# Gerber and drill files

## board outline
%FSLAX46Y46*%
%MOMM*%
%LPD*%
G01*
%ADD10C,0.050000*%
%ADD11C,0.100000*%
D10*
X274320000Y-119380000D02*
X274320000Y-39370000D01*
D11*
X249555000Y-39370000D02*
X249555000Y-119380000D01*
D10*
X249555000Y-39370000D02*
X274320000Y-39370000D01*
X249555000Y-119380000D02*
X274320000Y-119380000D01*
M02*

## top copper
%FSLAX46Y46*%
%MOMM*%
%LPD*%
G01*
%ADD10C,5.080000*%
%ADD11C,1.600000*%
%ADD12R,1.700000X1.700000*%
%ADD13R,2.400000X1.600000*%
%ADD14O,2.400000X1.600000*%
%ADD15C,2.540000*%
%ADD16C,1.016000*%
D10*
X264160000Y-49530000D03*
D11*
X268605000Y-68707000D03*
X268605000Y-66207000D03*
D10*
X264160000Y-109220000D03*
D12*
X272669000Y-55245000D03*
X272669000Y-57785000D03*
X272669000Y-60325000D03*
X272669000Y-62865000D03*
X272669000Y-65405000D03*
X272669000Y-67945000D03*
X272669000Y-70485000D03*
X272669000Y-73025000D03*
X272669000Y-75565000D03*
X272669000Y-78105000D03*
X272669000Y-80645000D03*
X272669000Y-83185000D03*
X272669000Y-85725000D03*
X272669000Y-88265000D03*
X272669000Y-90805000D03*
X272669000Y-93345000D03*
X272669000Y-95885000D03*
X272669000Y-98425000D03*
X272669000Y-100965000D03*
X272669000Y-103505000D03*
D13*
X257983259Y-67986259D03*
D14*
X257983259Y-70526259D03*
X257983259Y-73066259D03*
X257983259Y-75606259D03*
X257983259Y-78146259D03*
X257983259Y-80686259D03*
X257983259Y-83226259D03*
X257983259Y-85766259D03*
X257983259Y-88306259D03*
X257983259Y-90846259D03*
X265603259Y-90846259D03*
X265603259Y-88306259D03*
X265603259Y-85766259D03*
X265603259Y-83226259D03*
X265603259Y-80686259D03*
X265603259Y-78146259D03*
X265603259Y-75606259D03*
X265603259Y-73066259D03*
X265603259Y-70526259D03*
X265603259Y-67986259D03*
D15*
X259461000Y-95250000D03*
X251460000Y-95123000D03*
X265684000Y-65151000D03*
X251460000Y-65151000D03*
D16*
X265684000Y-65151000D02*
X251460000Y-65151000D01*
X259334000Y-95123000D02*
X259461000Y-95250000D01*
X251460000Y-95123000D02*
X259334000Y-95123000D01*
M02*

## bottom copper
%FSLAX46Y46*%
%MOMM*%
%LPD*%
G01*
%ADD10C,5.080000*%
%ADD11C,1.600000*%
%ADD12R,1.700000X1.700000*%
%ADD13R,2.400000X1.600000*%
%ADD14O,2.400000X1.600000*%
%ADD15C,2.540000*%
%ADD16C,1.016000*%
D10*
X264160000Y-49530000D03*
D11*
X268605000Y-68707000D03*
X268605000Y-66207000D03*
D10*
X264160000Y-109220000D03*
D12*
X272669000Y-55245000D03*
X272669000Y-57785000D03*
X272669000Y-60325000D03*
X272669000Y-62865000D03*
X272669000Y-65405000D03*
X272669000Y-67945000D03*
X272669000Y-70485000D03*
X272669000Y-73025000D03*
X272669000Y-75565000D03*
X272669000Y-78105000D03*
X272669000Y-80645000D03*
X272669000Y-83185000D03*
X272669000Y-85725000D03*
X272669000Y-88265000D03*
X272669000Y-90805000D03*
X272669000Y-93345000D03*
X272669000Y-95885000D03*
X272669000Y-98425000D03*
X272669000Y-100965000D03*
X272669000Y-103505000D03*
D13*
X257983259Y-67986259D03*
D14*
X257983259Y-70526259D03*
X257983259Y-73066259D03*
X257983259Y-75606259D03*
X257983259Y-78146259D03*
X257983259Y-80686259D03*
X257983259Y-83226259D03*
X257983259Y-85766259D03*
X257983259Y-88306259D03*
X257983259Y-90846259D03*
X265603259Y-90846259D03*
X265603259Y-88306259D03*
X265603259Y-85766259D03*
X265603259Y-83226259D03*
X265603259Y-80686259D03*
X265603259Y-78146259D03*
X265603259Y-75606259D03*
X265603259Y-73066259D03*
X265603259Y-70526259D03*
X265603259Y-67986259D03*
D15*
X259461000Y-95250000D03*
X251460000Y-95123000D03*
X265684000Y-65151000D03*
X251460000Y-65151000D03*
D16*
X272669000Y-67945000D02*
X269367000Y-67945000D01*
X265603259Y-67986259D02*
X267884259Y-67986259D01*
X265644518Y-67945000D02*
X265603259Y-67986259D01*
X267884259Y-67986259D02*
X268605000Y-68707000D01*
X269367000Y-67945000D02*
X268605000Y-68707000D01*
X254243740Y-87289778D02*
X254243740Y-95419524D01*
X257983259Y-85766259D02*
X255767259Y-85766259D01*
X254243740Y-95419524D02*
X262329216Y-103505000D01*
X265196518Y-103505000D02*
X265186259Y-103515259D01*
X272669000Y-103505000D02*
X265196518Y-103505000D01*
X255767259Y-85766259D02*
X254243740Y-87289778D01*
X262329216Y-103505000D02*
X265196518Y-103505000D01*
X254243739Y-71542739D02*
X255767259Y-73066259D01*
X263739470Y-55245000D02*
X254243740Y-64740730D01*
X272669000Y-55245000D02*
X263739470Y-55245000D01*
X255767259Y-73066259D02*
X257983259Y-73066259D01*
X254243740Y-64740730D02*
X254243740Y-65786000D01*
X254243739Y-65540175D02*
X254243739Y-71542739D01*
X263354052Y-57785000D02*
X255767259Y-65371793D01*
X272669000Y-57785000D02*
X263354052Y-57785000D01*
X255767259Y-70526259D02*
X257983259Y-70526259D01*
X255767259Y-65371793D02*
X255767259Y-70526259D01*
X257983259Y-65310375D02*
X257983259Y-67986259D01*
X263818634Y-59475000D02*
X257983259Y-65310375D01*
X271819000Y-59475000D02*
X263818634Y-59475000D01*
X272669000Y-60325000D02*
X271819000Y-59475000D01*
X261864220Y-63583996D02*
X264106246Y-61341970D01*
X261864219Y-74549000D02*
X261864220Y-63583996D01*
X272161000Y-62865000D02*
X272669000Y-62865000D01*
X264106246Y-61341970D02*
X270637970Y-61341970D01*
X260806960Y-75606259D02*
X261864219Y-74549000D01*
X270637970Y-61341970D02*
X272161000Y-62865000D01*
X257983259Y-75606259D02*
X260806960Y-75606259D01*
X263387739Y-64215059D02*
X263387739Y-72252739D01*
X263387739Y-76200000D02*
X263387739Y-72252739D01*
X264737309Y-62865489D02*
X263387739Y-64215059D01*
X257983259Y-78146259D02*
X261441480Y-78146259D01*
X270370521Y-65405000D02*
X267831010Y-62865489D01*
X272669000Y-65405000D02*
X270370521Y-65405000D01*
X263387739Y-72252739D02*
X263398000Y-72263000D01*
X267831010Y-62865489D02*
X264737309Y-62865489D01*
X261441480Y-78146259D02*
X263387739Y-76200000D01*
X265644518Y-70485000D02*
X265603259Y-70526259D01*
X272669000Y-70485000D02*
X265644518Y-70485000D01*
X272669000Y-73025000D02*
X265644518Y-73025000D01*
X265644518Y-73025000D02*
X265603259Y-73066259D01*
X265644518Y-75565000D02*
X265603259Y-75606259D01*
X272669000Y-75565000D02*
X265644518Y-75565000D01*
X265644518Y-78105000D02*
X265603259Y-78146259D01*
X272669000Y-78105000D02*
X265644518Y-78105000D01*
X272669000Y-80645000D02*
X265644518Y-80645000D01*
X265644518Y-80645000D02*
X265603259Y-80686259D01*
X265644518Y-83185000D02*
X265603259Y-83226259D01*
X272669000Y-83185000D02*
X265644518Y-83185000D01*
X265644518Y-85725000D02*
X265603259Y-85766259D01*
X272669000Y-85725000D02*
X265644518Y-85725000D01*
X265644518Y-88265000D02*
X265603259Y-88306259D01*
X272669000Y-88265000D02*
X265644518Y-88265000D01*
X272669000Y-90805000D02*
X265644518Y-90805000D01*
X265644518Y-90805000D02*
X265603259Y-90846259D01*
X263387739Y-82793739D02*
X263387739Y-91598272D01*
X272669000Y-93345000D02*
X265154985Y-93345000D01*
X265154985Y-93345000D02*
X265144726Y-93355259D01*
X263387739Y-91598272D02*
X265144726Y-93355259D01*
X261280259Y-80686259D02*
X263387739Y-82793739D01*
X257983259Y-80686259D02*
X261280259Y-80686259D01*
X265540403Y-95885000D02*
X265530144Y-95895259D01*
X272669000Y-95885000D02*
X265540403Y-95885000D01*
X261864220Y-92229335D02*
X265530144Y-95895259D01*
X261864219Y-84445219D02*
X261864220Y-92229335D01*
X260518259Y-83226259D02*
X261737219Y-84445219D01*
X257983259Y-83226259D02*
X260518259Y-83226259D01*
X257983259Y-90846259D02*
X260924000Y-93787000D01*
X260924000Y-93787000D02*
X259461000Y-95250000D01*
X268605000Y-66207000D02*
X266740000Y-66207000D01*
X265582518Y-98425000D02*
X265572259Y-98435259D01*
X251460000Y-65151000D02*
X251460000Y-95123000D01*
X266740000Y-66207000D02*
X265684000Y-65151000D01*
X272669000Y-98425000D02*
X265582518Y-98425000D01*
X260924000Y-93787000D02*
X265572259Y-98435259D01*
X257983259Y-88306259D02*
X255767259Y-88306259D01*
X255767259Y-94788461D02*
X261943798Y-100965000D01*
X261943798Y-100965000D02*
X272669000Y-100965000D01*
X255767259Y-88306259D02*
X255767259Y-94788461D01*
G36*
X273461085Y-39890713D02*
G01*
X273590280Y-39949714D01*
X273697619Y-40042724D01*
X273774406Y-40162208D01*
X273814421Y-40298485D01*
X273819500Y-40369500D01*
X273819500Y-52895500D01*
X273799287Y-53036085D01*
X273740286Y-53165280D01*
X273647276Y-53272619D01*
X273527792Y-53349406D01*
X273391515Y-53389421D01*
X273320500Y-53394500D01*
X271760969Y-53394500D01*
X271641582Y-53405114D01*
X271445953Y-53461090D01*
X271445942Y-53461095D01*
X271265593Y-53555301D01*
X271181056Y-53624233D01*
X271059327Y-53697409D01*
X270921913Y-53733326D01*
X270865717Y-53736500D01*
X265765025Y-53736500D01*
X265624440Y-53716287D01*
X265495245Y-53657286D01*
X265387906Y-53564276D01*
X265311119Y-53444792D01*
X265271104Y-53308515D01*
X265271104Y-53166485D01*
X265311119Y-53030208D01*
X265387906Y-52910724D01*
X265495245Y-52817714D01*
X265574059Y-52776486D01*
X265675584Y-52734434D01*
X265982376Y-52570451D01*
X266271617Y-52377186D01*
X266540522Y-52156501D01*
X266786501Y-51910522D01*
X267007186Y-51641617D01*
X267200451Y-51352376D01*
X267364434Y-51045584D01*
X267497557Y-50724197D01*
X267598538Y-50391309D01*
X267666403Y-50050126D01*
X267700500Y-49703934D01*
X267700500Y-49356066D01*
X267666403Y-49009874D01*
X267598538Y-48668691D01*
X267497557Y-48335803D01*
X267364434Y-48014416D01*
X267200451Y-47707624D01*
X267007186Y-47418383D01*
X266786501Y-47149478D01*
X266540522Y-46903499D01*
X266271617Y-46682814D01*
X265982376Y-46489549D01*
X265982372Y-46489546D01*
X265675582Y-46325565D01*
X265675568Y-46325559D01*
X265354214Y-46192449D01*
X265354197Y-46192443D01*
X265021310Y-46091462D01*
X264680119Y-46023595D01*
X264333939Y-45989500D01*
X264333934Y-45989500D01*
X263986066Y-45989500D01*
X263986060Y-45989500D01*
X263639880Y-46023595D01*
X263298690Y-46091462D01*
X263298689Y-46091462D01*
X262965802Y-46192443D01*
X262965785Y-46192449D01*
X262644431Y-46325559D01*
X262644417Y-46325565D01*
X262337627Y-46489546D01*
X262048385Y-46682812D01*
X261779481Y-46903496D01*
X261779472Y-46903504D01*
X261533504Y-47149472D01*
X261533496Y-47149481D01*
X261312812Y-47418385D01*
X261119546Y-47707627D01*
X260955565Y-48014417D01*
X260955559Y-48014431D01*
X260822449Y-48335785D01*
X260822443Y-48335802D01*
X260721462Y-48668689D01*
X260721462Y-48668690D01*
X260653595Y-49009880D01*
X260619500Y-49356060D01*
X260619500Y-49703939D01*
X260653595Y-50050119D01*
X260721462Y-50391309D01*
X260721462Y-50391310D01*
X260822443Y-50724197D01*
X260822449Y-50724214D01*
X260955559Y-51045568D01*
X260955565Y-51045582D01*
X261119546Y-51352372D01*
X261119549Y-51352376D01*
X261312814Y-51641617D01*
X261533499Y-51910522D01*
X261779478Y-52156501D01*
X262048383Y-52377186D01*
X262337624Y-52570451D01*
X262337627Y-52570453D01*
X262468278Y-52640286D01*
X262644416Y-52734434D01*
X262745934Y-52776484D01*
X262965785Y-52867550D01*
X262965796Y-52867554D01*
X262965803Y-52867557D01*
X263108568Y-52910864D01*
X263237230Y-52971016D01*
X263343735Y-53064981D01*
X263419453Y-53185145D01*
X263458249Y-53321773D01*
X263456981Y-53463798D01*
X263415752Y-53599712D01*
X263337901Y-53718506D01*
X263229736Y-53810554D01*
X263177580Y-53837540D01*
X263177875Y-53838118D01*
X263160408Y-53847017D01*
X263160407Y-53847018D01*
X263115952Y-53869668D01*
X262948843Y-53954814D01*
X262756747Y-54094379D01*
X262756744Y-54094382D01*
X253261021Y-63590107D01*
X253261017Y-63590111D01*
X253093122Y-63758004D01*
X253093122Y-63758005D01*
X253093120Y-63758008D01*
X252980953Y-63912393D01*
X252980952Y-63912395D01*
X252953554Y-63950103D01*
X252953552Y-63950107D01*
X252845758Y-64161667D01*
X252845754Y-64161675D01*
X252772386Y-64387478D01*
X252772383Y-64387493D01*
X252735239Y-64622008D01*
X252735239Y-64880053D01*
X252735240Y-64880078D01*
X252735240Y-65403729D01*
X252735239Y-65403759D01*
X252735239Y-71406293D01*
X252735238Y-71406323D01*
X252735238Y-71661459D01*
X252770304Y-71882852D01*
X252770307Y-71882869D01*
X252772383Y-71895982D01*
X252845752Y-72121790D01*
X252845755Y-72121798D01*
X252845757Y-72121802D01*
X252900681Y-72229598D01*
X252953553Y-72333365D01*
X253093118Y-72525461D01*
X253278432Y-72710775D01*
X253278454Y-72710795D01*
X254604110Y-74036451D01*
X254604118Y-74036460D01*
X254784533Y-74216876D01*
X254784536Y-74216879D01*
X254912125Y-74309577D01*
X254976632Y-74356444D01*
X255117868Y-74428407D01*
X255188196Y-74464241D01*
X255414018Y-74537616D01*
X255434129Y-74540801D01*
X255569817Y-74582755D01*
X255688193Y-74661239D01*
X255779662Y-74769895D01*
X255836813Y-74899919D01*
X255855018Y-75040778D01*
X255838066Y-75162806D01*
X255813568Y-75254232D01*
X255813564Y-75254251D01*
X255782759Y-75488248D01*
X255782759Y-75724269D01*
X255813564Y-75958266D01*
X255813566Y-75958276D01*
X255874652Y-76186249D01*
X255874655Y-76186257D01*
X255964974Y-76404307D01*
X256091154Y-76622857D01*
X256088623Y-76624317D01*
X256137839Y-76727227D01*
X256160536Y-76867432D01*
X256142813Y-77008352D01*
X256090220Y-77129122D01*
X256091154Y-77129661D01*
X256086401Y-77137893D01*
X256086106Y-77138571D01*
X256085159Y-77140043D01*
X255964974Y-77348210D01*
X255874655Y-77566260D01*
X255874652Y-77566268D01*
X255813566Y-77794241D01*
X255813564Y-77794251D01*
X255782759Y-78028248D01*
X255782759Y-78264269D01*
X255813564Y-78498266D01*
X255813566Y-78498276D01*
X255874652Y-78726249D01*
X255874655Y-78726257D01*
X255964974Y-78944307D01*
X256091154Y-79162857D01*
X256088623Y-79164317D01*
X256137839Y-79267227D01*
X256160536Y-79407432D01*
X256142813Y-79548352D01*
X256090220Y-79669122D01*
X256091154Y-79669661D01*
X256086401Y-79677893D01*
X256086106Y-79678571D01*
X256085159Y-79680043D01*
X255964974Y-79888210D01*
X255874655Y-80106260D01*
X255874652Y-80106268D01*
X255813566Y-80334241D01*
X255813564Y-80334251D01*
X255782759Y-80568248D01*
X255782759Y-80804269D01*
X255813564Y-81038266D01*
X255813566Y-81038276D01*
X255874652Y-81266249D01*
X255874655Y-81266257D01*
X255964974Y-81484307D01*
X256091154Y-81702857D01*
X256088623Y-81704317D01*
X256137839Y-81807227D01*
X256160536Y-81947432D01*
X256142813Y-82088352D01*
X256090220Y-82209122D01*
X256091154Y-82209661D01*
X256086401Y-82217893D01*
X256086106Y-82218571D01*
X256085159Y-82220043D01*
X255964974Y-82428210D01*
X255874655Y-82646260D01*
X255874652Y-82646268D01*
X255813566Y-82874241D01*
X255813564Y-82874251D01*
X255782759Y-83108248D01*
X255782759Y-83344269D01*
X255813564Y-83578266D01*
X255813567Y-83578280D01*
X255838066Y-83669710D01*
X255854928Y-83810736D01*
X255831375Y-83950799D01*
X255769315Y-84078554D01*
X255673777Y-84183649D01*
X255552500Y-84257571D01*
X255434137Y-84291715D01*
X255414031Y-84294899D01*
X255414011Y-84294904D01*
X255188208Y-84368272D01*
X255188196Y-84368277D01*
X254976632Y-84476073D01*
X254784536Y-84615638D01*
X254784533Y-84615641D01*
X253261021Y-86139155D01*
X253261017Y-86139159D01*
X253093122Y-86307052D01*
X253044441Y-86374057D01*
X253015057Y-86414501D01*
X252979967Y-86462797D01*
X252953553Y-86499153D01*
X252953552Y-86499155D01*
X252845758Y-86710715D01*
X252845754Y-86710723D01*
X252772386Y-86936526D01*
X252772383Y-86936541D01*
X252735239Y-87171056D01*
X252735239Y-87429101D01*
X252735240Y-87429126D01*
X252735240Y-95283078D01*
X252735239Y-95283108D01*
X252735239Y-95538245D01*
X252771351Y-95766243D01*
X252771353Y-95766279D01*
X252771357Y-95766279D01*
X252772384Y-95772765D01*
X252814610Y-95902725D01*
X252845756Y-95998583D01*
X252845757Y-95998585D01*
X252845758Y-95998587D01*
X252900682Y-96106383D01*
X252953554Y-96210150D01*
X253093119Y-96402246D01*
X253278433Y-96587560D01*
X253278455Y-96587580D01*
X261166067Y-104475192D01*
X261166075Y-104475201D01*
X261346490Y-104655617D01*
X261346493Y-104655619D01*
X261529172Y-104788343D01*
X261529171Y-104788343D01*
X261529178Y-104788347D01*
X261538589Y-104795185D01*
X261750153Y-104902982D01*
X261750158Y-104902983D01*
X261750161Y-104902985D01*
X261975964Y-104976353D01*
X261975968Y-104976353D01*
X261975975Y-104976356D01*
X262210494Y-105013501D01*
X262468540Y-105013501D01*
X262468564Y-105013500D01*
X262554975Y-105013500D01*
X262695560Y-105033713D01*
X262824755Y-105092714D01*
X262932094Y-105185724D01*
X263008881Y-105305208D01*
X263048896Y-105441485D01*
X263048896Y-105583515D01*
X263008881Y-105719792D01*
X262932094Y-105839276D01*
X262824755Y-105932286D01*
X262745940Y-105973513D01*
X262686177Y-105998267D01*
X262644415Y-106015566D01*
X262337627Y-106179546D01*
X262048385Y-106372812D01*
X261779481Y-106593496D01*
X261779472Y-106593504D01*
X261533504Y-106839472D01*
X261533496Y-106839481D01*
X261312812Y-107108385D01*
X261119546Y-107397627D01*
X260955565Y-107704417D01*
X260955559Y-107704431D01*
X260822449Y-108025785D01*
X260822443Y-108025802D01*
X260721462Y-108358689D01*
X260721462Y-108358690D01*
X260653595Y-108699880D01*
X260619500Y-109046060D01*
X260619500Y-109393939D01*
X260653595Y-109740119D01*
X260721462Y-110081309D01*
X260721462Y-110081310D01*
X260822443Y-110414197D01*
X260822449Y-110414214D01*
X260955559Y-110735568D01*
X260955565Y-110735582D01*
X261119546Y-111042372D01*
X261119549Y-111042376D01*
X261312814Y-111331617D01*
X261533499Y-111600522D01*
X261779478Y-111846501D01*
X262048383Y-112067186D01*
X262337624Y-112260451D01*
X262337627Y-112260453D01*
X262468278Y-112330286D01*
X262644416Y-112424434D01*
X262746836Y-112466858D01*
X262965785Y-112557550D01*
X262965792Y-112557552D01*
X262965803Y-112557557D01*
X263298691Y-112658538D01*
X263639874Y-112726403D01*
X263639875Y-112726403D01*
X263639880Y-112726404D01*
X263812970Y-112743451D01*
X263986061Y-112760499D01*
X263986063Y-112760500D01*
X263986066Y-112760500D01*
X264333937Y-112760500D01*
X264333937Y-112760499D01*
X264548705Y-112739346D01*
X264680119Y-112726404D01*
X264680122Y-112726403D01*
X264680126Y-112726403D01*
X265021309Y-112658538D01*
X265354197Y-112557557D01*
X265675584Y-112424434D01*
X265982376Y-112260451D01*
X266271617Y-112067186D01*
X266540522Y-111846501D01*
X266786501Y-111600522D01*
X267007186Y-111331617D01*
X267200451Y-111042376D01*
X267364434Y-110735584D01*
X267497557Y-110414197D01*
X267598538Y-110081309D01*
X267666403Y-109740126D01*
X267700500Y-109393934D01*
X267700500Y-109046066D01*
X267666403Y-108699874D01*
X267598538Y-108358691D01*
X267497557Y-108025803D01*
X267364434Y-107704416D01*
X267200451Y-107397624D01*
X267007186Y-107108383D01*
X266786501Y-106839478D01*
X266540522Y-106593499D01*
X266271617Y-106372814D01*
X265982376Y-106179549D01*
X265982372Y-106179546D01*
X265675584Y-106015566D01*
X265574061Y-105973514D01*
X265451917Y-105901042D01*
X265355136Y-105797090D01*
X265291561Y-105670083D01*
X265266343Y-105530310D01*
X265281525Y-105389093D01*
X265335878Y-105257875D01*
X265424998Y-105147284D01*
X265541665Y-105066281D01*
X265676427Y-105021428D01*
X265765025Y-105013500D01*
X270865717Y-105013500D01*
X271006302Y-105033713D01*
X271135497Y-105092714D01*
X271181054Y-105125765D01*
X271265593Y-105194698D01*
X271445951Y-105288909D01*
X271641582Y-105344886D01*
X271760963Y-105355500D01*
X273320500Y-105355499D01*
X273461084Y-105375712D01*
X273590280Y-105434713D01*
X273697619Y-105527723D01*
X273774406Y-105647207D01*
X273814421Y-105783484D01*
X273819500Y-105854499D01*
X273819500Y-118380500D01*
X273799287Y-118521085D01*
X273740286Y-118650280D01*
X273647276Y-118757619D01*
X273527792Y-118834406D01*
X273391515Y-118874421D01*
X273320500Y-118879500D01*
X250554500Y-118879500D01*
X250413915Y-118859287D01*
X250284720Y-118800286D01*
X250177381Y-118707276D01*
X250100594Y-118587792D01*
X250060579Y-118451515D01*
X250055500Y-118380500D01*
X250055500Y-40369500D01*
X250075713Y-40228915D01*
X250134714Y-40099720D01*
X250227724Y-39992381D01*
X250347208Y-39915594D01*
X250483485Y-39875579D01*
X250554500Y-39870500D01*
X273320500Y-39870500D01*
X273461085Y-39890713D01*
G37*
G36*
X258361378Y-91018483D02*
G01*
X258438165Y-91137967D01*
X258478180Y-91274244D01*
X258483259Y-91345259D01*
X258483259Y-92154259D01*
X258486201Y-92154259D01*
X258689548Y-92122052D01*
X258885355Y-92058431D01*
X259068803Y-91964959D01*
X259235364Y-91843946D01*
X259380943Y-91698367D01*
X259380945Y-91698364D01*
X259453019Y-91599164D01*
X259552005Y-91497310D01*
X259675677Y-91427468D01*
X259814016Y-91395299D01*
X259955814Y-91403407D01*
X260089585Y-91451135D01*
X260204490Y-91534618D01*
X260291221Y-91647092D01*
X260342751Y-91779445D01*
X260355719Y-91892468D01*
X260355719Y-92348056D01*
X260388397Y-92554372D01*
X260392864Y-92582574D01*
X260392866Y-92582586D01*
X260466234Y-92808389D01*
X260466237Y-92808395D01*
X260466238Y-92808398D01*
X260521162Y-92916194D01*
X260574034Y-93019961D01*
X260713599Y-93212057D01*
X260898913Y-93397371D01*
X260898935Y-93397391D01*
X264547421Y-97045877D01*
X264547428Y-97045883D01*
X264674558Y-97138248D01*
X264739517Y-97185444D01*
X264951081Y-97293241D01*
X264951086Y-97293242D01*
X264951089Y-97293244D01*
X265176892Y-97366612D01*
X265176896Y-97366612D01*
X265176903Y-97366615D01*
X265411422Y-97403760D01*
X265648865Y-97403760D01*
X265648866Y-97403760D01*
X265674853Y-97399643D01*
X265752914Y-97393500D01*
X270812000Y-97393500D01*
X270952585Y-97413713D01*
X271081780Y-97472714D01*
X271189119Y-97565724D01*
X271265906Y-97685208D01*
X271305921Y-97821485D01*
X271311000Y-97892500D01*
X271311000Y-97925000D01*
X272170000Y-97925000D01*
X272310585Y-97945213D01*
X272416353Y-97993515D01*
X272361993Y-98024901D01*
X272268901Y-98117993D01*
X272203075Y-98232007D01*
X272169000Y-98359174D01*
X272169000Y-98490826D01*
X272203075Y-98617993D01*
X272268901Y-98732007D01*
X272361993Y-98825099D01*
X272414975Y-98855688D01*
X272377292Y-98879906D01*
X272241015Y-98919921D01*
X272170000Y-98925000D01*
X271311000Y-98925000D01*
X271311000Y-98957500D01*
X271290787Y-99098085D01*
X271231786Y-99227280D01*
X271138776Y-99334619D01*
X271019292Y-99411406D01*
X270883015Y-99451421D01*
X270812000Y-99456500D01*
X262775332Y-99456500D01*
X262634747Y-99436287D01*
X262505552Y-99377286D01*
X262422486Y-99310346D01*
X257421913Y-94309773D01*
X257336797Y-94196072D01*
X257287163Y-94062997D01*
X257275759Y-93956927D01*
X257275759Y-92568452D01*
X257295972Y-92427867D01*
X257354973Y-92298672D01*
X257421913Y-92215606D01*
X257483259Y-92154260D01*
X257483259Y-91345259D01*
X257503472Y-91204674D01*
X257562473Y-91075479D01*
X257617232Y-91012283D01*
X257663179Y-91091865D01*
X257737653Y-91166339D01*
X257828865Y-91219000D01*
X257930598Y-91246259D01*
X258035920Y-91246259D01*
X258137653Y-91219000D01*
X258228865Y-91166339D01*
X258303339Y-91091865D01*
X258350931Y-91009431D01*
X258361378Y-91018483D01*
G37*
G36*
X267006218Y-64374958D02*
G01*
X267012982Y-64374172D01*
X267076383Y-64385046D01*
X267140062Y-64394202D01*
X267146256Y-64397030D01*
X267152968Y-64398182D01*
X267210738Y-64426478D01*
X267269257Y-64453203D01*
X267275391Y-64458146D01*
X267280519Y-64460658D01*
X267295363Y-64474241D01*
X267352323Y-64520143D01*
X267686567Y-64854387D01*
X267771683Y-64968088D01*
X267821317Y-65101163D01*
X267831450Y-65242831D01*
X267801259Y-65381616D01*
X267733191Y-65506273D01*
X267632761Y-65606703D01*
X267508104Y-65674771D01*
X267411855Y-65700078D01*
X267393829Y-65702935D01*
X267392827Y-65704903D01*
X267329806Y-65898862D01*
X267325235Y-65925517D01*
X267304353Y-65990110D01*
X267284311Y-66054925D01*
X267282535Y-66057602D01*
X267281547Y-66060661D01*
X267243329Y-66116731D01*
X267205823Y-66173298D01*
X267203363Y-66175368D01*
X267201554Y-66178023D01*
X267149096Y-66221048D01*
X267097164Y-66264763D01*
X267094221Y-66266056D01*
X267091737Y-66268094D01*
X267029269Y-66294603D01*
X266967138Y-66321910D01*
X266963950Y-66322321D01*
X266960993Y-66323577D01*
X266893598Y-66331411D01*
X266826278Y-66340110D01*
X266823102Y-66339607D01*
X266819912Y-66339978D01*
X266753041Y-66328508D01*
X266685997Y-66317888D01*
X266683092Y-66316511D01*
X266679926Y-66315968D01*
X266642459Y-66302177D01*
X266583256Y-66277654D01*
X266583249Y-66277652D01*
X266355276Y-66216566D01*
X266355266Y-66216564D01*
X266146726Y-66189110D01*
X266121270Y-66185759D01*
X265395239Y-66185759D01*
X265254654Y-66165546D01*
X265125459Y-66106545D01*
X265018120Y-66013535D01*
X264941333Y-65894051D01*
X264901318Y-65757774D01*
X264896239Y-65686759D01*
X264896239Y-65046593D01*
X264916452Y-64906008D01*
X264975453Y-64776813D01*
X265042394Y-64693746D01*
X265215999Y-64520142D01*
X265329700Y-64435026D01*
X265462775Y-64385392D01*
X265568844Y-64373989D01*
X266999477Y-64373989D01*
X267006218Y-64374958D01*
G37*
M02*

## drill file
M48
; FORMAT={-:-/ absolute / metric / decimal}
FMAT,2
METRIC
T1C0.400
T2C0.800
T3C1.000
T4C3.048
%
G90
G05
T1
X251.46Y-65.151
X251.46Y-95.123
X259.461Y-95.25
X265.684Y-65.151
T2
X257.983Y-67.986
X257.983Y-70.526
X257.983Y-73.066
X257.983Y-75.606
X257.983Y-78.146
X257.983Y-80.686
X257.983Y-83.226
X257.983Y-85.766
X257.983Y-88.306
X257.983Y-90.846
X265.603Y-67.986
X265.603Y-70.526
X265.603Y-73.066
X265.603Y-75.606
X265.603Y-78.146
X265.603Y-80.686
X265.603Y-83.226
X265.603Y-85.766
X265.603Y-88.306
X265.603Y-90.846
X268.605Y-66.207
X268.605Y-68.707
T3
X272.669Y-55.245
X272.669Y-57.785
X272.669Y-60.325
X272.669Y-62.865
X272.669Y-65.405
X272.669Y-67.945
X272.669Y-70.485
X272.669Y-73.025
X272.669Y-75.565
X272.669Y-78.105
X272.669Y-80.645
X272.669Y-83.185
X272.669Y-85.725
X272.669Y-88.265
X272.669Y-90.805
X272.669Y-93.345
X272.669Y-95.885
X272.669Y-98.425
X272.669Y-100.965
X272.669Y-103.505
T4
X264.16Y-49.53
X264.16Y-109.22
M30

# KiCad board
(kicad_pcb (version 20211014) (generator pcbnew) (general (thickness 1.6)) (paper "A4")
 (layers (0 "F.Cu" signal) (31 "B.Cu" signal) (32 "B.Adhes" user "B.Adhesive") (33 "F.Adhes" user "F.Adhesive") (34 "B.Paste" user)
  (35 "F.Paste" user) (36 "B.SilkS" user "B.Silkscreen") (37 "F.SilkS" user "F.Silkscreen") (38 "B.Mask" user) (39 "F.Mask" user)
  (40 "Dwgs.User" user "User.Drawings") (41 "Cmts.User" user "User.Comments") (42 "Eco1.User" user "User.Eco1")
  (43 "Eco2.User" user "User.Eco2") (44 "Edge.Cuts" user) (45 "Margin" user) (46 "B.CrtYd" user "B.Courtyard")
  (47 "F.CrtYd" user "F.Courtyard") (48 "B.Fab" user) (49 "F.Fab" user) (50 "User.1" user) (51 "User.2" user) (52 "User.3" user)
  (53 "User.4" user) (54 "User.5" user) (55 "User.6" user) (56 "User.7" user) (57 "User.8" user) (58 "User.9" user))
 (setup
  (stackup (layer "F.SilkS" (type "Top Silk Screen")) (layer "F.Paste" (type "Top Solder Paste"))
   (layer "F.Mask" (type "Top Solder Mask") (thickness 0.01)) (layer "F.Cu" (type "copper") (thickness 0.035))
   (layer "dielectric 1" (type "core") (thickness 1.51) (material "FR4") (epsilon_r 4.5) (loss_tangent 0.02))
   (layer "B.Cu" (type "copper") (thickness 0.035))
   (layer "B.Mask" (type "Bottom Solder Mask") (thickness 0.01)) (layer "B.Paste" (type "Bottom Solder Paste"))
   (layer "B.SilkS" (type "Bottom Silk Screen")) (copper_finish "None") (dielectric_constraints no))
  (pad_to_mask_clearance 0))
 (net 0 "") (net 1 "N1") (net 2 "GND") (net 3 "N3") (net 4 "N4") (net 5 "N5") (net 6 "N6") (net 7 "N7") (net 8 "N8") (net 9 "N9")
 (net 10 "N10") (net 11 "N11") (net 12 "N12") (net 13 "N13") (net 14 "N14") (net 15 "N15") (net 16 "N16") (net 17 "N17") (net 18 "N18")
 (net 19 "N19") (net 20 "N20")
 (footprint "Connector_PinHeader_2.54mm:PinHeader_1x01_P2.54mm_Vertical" (layer "F.Cu") (at 264.16 49.53)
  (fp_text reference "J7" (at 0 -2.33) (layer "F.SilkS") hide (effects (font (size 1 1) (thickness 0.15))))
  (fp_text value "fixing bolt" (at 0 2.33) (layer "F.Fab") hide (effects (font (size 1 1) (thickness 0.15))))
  (pad "" thru_hole circle locked (at 0 0) (size 5.08 5.08) (drill 3.048) (layers *.Cu *.Mask)))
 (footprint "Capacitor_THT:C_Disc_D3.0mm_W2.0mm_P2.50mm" (layer "F.Cu") (at 268.605 68.707 90)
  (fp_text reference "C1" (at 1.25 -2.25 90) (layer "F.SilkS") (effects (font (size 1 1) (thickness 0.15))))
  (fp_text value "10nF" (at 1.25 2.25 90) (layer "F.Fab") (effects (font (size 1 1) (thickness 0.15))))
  (pad "1" thru_hole circle (at 0 0 90) (size 1.6 1.6) (drill 0.8) (layers *.Cu *.Mask) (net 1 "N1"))
  (pad "2" thru_hole circle (at 2.5 0 90) (size 1.6 1.6) (drill 0.8) (layers *.Cu *.Mask) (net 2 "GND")))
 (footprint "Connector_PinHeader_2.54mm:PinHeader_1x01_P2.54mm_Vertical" (layer "F.Cu") (at 264.16 109.22)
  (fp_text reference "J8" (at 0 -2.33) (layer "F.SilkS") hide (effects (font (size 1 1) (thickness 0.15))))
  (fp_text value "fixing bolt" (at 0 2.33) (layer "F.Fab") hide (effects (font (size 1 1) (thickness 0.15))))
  (pad "1" thru_hole circle locked (at 0 0) (size 5.08 5.08) (drill 3.048) (layers *.Cu *.Mask)))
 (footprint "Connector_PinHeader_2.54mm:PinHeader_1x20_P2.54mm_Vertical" (layer "F.Cu") (at 272.669 55.245)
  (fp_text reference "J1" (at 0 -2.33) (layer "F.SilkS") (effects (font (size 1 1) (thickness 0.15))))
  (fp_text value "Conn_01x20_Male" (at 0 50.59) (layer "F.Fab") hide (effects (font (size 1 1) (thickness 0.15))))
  (pad "1" thru_hole rect (at 0 0) (size 1.7 1.7) (drill 1) (layers *.Cu *.Mask) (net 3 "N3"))
  (pad "2" thru_hole rect (at 0 2.54) (size 1.7 1.7) (drill 1) (layers *.Cu *.Mask) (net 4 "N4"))
  (pad "3" thru_hole rect (at 0 5.08) (size 1.7 1.7) (drill 1) (layers *.Cu *.Mask) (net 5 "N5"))
  (pad "4" thru_hole rect (at 0 7.62) (size 1.7 1.7) (drill 1) (layers *.Cu *.Mask) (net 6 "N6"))
  (pad "5" thru_hole rect (at 0 10.16) (size 1.7 1.7) (drill 1) (layers *.Cu *.Mask) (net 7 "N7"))
  (pad "6" thru_hole rect (at 0 12.7) (size 1.7 1.7) (drill 1) (layers *.Cu *.Mask) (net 1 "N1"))
  (pad "7" thru_hole rect (at 0 15.24) (size 1.7 1.7) (drill 1) (layers *.Cu *.Mask) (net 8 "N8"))
  (pad "8" thru_hole rect (at 0 17.78) (size 1.7 1.7) (drill 1) (layers *.Cu *.Mask) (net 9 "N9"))
  (pad "9" thru_hole rect (at 0 20.32) (size 1.7 1.7) (drill 1) (layers *.Cu *.Mask) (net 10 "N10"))
  (pad "10" thru_hole rect (at 0 22.86) (size 1.7 1.7) (drill 1) (layers *.Cu *.Mask) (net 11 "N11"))
  (pad "11" thru_hole rect (at 0 25.4) (size 1.7 1.7) (drill 1) (layers *.Cu *.Mask) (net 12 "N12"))
  (pad "12" thru_hole rect (at 0 27.94) (size 1.7 1.7) (drill 1) (layers *.Cu *.Mask) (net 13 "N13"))
  (pad "13" thru_hole rect (at 0 30.48) (size 1.7 1.7) (drill 1) (layers *.Cu *.Mask) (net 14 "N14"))
  (pad "14" thru_hole rect (at 0 33.02) (size 1.7 1.7) (drill 1) (layers *.Cu *.Mask) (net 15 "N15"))
  (pad "15" thru_hole rect (at 0 35.56) (size 1.7 1.7) (drill 1) (layers *.Cu *.Mask) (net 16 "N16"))
  (pad "16" thru_hole rect (at 0 38.1) (size 1.7 1.7) (drill 1) (layers *.Cu *.Mask) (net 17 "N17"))
  (pad "17" thru_hole rect (at 0 40.64) (size 1.7 1.7) (drill 1) (layers *.Cu *.Mask) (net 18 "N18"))
  (pad "18" thru_hole rect (at 0 43.18) (size 1.7 1.7) (drill 1) (layers *.Cu *.Mask) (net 2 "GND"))
  (pad "19" thru_hole rect (at 0 45.72) (size 1.7 1.7) (drill 1) (layers *.Cu *.Mask) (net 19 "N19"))
  (pad "20" thru_hole rect (at 0 48.26) (size 1.7 1.7) (drill 1) (layers *.Cu *.Mask) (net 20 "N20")))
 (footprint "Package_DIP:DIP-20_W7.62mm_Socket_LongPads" (layer "F.Cu") (at 257.983259 67.986259)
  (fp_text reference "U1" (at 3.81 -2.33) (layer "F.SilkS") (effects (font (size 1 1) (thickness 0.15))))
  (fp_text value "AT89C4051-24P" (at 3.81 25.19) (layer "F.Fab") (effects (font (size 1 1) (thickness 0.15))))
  (pad "1" thru_hole rect (at 0 0) (size 2.4 1.6) (drill 0.8) (layers *.Cu *.Mask) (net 5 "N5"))
  (pad "2" thru_hole oval (at 0 2.54) (size 2.4 1.6) (drill 0.8) (layers *.Cu *.Mask) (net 4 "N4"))
  (pad "3" thru_hole oval (at 0 5.08) (size 2.4 1.6) (drill 0.8) (layers *.Cu *.Mask) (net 3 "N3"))
  (pad "4" thru_hole oval (at 0 7.62) (size 2.4 1.6) (drill 0.8) (layers *.Cu *.Mask) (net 6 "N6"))
  (pad "5" thru_hole oval (at 0 10.16) (size 2.4 1.6) (drill 0.8) (layers *.Cu *.Mask) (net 7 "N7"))
  (pad "6" thru_hole oval (at 0 12.7) (size 2.4 1.6) (drill 0.8) (layers *.Cu *.Mask) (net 17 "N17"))
  (pad "7" thru_hole oval (at 0 15.24) (size 2.4 1.6) (drill 0.8) (layers *.Cu *.Mask) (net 18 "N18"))
  (pad "8" thru_hole oval (at 0 17.78) (size 2.4 1.6) (drill 0.8) (layers *.Cu *.Mask) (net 20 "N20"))
  (pad "9" thru_hole oval (at 0 20.32) (size 2.4 1.6) (drill 0.8) (layers *.Cu *.Mask) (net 19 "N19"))
  (pad "10" thru_hole oval (at 0 22.86) (size 2.4 1.6) (drill 0.8) (layers *.Cu *.Mask) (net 2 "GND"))
  (pad "11" thru_hole oval (at 7.62 22.86) (size 2.4 1.6) (drill 0.8) (layers *.Cu *.Mask) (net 16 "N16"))
  (pad "12" thru_hole oval (at 7.62 20.32) (size 2.4 1.6) (drill 0.8) (layers *.Cu *.Mask) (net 15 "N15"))
  (pad "13" thru_hole oval (at 7.62 17.78) (size 2.4 1.6) (drill 0.8) (layers *.Cu *.Mask) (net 14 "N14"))
  (pad "14" thru_hole oval (at 7.62 15.24) (size 2.4 1.6) (drill 0.8) (layers *.Cu *.Mask) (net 13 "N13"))
  (pad "15" thru_hole oval (at 7.62 12.7) (size 2.4 1.6) (drill 0.8) (layers *.Cu *.Mask) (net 12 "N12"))
  (pad "16" thru_hole oval (at 7.62 10.16) (size 2.4 1.6) (drill 0.8) (layers *.Cu *.Mask) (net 11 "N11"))
  (pad "17" thru_hole oval (at 7.62 7.62) (size 2.4 1.6) (drill 0.8) (layers *.Cu *.Mask) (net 10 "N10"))
  (pad "18" thru_hole oval (at 7.62 5.08) (size 2.4 1.6) (drill 0.8) (layers *.Cu *.Mask) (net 9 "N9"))
  (pad "19" thru_hole oval (at 7.62 2.54) (size 2.4 1.6) (drill 0.8) (layers *.Cu *.Mask) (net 8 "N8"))
  (pad "20" thru_hole oval (at 7.62 0) (size 2.4 1.6) (drill 0.8) (layers *.Cu *.Mask) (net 1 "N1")))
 (gr_line (start 274.32 119.38) (end 274.32 39.37) (layer "Edge.Cuts") (width 0.05))
 (gr_line (start 249.555 39.37) (end 249.555 119.38) (layer "Edge.Cuts") (width 0.1))
 (gr_line (start 249.555 39.37) (end 274.32 39.37) (layer "Edge.Cuts") (width 0.05))
 (gr_line (start 249.555 119.38) (end 274.32 119.38) (layer "Edge.Cuts") (width 0.05))
 (segment (start 272.669 67.945) (end 269.367 67.945) (width 1.016) (layer "B.Cu") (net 1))
 (segment (start 265.603259 67.986259) (end 267.884259 67.986259) (width 1.016) (layer "B.Cu") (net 1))
 (segment (start 265.644518 67.945) (end 265.603259 67.986259) (width 1.016) (layer "B.Cu") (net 1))
 (segment (start 267.884259 67.986259) (end 268.605 68.707) (width 1.016) (layer "B.Cu") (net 1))
 (segment (start 269.367 67.945) (end 268.605 68.707) (width 1.016) (layer "B.Cu") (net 1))
 (segment (start 254.24374 87.289778) (end 254.24374 95.419524) (width 1.016) (layer "B.Cu") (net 20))
 (segment (start 257.983259 85.766259) (end 255.767259 85.766259) (width 1.016) (layer "B.Cu") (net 20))
 (segment (start 254.24374 95.419524) (end 262.329216 103.505) (width 1.016) (layer "B.Cu") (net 20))
 (segment (start 265.196518 103.505) (end 265.186259 103.515259) (width 1.016) (layer "B.Cu") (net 20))
 (segment (start 272.669 103.505) (end 265.196518 103.505) (width 1.016) (layer "B.Cu") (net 20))
 (segment (start 255.767259 85.766259) (end 254.24374 87.289778) (width 1.016) (layer "B.Cu") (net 20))
 (segment (start 262.329216 103.505) (end 265.196518 103.505) (width 1.016) (layer "B.Cu") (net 20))
 (segment (start 254.243739 71.542739) (end 255.767259 73.066259) (width 1.016) (layer "B.Cu") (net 3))
 (segment (start 263.73947 55.245) (end 254.24374 64.74073) (width 1.016) (layer "B.Cu") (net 3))
 (segment (start 272.669 55.245) (end 263.73947 55.245) (width 1.016) (layer "B.Cu") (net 3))
 (segment (start 255.767259 73.066259) (end 257.983259 73.066259) (width 1.016) (layer "B.Cu") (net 3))
 (segment (start 254.24374 64.74073) (end 254.24374 65.786) (width 1.016) (layer "B.Cu") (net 3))
 (segment (start 254.243739 65.540175) (end 254.243739 71.542739) (width 1.016) (layer "B.Cu") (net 3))
 (segment (start 263.354052 57.785) (end 255.767259 65.371793) (width 1.016) (layer "B.Cu") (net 4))
 (segment (start 272.669 57.785) (end 263.354052 57.785) (width 1.016) (layer "B.Cu") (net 4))
 (segment (start 255.767259 70.526259) (end 257.983259 70.526259) (width 1.016) (layer "B.Cu") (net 4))
 (segment (start 255.767259 65.371793) (end 255.767259 70.526259) (width 1.016) (layer "B.Cu") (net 4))
 (segment (start 257.983259 65.310375) (end 257.983259 67.986259) (width 1.016) (layer "B.Cu") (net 5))
 (segment (start 263.818634 59.475) (end 257.983259 65.310375) (width 1.016) (layer "B.Cu") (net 5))
 (segment (start 271.819 59.475) (end 263.818634 59.475) (width 1.016) (layer "B.Cu") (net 5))
 (segment (start 272.669 60.325) (end 271.819 59.475) (width 1.016) (layer "B.Cu") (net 5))
 (segment (start 261.86422 63.583996) (end 264.106246 61.34197) (width 1.016) (layer "B.Cu") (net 6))
 (segment (start 261.864219 74.549) (end 261.86422 63.583996) (width 1.016) (layer "B.Cu") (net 6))
 (segment (start 272.161 62.865) (end 272.669 62.865) (width 1.016) (layer "B.Cu") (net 6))
 (segment (start 264.106246 61.34197) (end 270.63797 61.34197) (width 1.016) (layer "B.Cu") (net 6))
 (segment (start 260.80696 75.606259) (end 261.864219 74.549) (width 1.016) (layer "B.Cu") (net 6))
 (segment (start 270.63797 61.34197) (end 272.161 62.865) (width 1.016) (layer "B.Cu") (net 6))
 (segment (start 257.983259 75.606259) (end 260.80696 75.606259) (width 1.016) (layer "B.Cu") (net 6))
 (segment (start 263.387739 64.215059) (end 263.387739 72.252739) (width 1.016) (layer "B.Cu") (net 7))
 (segment (start 263.387739 76.2) (end 263.387739 72.252739) (width 1.016) (layer "B.Cu") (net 7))
 (segment (start 264.737309 62.865489) (end 263.387739 64.215059) (width 1.016) (layer "B.Cu") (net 7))
 (segment (start 257.983259 78.146259) (end 261.44148 78.146259) (width 1.016) (layer "B.Cu") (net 7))
 (segment (start 270.370521 65.405) (end 267.83101 62.865489) (width 1.016) (layer "B.Cu") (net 7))
 (segment (start 272.669 65.405) (end 270.370521 65.405) (width 1.016) (layer "B.Cu") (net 7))
 (segment (start 263.387739 72.252739) (end 263.398 72.263) (width 1.016) (layer "B.Cu") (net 7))
 (segment (start 267.83101 62.865489) (end 264.737309 62.865489) (width 1.016) (layer "B.Cu") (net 7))
 (segment (start 261.44148 78.146259) (end 263.387739 76.2) (width 1.016) (layer "B.Cu") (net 7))
 (segment (start 265.644518 70.485) (end 265.603259 70.526259) (width 1.016) (layer "B.Cu") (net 8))
 (segment (start 272.669 70.485) (end 265.644518 70.485) (width 1.016) (layer "B.Cu") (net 8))
 (segment (start 272.669 73.025) (end 265.644518 73.025) (width 1.016) (layer "B.Cu") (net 9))
 (segment (start 265.644518 73.025) (end 265.603259 73.066259) (width 1.016) (layer "B.Cu") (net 9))
 (segment (start 265.644518 75.565) (end 265.603259 75.606259) (width 1.016) (layer "B.Cu") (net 10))
 (segment (start 272.669 75.565) (end 265.644518 75.565) (width 1.016) (layer "B.Cu") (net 10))
 (segment (start 265.644518 78.105) (end 265.603259 78.146259) (width 1.016) (layer "B.Cu") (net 11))
 (segment (start 272.669 78.105) (end 265.644518 78.105) (width 1.016) (layer "B.Cu") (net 11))
 (segment (start 272.669 80.645) (end 265.644518 80.645) (width 1.016) (layer "B.Cu") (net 12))
 (segment (start 265.644518 80.645) (end 265.603259 80.686259) (width 1.016) (layer "B.Cu") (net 12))
 (segment (start 265.644518 83.185) (end 265.603259 83.226259) (width 1.016) (layer "B.Cu") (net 13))
 (segment (start 272.669 83.185) (end 265.644518 83.185) (width 1.016) (layer "B.Cu") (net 13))
 (segment (start 265.644518 85.725) (end 265.603259 85.766259) (width 1.016) (layer "B.Cu") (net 14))
 (segment (start 272.669 85.725) (end 265.644518 85.725) (width 1.016) (layer "B.Cu") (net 14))
 (segment (start 265.644518 88.265) (end 265.603259 88.306259) (width 1.016) (layer "B.Cu") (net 15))
 (segment (start 272.669 88.265) (end 265.644518 88.265) (width 1.016) (layer "B.Cu") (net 15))
 (segment (start 272.669 90.805) (end 265.644518 90.805) (width 1.016) (layer "B.Cu") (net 16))
 (segment (start 265.644518 90.805) (end 265.603259 90.846259) (width 1.016) (layer "B.Cu") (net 16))
 (segment (start 263.387739 82.793739) (end 263.387739 91.598272) (width 1.016) (layer "B.Cu") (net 17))
 (segment (start 272.669 93.345) (end 265.154985 93.345) (width 1.016) (layer "B.Cu") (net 17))
 (segment (start 265.154985 93.345) (end 265.144726 93.355259) (width 1.016) (layer "B.Cu") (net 17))
 (segment (start 263.387739 91.598272) (end 265.144726 93.355259) (width 1.016) (layer "B.Cu") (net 17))
 (segment (start 261.280259 80.686259) (end 263.387739 82.793739) (width 1.016) (layer "B.Cu") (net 17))
 (segment (start 257.983259 80.686259) (end 261.280259 80.686259) (width 1.016) (layer "B.Cu") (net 17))
 (segment (start 265.540403 95.885) (end 265.530144 95.895259) (width 1.016) (layer "B.Cu") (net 18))
 (segment (start 272.669 95.885) (end 265.540403 95.885) (width 1.016) (layer "B.Cu") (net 18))
 (segment (start 261.86422 92.229335) (end 265.530144 95.895259) (width 1.016) (layer "B.Cu") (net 18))
 (segment (start 261.864219 84.445219) (end 261.86422 92.229335) (width 1.016) (layer "B.Cu") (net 18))
 (segment (start 260.518259 83.226259) (end 261.737219 84.445219) (width 1.016) (layer "B.Cu") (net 18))
 (segment (start 257.983259 83.226259) (end 260.518259 83.226259) (width 1.016) (layer "B.Cu") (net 18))
 (segment (start 265.684 65.151) (end 251.46 65.151) (width 1.016) (layer "F.Cu") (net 2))
 (segment (start 259.334 95.123) (end 259.461 95.25) (width 1.016) (layer "F.Cu") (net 2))
 (segment (start 251.46 95.123) (end 259.334 95.123) (width 1.016) (layer "F.Cu") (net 2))
 (via (at 259.461 95.25) (size 2.54) (drill 0.4) (layers "F.Cu" "B.Cu") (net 2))
 (via (at 251.46 95.123) (size 2.54) (drill 0.4) (layers "F.Cu" "B.Cu") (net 2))
 (via (at 265.684 65.151) (size 2.54) (drill 0.4) (layers "F.Cu" "B.Cu") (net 2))
 (via (at 251.46 65.151) (size 2.54) (drill 0.4) (layers "F.Cu" "B.Cu") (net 2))
 (segment (start 257.983259 90.846259) (end 260.924 93.787) (width 1.016) (layer "B.Cu") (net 2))
 (segment (start 260.924 93.787) (end 259.461 95.25) (width 1.016) (layer "B.Cu") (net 2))
 (segment (start 268.605 66.207) (end 266.74 66.207) (width 1.016) (layer "B.Cu") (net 2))
 (segment (start 265.582518 98.425) (end 265.572259 98.435259) (width 1.016) (layer "B.Cu") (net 2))
 (segment (start 251.46 65.151) (end 251.46 95.123) (width 1.016) (layer "B.Cu") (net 2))
 (segment (start 266.74 66.207) (end 265.684 65.151) (width 1.016) (layer "B.Cu") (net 2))
 (segment (start 272.669 98.425) (end 265.582518 98.425) (width 1.016) (layer "B.Cu") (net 2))
 (segment (start 260.924 93.787) (end 265.572259 98.435259) (width 1.016) (layer "B.Cu") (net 2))
 (segment (start 257.983259 88.306259) (end 255.767259 88.306259) (width 1.016) (layer "B.Cu") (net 19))
 (segment (start 255.767259 94.788461) (end 261.943798 100.965) (width 1.016) (layer "B.Cu") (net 19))
 (segment (start 261.943798 100.965) (end 272.669 100.965) (width 1.016) (layer "B.Cu") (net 19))
 (segment (start 255.767259 88.306259) (end 255.767259 94.788461) (width 1.016) (layer "B.Cu") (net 19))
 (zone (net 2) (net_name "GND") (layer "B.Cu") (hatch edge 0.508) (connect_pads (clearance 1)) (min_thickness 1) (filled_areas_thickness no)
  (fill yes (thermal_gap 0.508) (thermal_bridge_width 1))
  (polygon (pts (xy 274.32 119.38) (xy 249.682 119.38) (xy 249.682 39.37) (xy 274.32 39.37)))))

